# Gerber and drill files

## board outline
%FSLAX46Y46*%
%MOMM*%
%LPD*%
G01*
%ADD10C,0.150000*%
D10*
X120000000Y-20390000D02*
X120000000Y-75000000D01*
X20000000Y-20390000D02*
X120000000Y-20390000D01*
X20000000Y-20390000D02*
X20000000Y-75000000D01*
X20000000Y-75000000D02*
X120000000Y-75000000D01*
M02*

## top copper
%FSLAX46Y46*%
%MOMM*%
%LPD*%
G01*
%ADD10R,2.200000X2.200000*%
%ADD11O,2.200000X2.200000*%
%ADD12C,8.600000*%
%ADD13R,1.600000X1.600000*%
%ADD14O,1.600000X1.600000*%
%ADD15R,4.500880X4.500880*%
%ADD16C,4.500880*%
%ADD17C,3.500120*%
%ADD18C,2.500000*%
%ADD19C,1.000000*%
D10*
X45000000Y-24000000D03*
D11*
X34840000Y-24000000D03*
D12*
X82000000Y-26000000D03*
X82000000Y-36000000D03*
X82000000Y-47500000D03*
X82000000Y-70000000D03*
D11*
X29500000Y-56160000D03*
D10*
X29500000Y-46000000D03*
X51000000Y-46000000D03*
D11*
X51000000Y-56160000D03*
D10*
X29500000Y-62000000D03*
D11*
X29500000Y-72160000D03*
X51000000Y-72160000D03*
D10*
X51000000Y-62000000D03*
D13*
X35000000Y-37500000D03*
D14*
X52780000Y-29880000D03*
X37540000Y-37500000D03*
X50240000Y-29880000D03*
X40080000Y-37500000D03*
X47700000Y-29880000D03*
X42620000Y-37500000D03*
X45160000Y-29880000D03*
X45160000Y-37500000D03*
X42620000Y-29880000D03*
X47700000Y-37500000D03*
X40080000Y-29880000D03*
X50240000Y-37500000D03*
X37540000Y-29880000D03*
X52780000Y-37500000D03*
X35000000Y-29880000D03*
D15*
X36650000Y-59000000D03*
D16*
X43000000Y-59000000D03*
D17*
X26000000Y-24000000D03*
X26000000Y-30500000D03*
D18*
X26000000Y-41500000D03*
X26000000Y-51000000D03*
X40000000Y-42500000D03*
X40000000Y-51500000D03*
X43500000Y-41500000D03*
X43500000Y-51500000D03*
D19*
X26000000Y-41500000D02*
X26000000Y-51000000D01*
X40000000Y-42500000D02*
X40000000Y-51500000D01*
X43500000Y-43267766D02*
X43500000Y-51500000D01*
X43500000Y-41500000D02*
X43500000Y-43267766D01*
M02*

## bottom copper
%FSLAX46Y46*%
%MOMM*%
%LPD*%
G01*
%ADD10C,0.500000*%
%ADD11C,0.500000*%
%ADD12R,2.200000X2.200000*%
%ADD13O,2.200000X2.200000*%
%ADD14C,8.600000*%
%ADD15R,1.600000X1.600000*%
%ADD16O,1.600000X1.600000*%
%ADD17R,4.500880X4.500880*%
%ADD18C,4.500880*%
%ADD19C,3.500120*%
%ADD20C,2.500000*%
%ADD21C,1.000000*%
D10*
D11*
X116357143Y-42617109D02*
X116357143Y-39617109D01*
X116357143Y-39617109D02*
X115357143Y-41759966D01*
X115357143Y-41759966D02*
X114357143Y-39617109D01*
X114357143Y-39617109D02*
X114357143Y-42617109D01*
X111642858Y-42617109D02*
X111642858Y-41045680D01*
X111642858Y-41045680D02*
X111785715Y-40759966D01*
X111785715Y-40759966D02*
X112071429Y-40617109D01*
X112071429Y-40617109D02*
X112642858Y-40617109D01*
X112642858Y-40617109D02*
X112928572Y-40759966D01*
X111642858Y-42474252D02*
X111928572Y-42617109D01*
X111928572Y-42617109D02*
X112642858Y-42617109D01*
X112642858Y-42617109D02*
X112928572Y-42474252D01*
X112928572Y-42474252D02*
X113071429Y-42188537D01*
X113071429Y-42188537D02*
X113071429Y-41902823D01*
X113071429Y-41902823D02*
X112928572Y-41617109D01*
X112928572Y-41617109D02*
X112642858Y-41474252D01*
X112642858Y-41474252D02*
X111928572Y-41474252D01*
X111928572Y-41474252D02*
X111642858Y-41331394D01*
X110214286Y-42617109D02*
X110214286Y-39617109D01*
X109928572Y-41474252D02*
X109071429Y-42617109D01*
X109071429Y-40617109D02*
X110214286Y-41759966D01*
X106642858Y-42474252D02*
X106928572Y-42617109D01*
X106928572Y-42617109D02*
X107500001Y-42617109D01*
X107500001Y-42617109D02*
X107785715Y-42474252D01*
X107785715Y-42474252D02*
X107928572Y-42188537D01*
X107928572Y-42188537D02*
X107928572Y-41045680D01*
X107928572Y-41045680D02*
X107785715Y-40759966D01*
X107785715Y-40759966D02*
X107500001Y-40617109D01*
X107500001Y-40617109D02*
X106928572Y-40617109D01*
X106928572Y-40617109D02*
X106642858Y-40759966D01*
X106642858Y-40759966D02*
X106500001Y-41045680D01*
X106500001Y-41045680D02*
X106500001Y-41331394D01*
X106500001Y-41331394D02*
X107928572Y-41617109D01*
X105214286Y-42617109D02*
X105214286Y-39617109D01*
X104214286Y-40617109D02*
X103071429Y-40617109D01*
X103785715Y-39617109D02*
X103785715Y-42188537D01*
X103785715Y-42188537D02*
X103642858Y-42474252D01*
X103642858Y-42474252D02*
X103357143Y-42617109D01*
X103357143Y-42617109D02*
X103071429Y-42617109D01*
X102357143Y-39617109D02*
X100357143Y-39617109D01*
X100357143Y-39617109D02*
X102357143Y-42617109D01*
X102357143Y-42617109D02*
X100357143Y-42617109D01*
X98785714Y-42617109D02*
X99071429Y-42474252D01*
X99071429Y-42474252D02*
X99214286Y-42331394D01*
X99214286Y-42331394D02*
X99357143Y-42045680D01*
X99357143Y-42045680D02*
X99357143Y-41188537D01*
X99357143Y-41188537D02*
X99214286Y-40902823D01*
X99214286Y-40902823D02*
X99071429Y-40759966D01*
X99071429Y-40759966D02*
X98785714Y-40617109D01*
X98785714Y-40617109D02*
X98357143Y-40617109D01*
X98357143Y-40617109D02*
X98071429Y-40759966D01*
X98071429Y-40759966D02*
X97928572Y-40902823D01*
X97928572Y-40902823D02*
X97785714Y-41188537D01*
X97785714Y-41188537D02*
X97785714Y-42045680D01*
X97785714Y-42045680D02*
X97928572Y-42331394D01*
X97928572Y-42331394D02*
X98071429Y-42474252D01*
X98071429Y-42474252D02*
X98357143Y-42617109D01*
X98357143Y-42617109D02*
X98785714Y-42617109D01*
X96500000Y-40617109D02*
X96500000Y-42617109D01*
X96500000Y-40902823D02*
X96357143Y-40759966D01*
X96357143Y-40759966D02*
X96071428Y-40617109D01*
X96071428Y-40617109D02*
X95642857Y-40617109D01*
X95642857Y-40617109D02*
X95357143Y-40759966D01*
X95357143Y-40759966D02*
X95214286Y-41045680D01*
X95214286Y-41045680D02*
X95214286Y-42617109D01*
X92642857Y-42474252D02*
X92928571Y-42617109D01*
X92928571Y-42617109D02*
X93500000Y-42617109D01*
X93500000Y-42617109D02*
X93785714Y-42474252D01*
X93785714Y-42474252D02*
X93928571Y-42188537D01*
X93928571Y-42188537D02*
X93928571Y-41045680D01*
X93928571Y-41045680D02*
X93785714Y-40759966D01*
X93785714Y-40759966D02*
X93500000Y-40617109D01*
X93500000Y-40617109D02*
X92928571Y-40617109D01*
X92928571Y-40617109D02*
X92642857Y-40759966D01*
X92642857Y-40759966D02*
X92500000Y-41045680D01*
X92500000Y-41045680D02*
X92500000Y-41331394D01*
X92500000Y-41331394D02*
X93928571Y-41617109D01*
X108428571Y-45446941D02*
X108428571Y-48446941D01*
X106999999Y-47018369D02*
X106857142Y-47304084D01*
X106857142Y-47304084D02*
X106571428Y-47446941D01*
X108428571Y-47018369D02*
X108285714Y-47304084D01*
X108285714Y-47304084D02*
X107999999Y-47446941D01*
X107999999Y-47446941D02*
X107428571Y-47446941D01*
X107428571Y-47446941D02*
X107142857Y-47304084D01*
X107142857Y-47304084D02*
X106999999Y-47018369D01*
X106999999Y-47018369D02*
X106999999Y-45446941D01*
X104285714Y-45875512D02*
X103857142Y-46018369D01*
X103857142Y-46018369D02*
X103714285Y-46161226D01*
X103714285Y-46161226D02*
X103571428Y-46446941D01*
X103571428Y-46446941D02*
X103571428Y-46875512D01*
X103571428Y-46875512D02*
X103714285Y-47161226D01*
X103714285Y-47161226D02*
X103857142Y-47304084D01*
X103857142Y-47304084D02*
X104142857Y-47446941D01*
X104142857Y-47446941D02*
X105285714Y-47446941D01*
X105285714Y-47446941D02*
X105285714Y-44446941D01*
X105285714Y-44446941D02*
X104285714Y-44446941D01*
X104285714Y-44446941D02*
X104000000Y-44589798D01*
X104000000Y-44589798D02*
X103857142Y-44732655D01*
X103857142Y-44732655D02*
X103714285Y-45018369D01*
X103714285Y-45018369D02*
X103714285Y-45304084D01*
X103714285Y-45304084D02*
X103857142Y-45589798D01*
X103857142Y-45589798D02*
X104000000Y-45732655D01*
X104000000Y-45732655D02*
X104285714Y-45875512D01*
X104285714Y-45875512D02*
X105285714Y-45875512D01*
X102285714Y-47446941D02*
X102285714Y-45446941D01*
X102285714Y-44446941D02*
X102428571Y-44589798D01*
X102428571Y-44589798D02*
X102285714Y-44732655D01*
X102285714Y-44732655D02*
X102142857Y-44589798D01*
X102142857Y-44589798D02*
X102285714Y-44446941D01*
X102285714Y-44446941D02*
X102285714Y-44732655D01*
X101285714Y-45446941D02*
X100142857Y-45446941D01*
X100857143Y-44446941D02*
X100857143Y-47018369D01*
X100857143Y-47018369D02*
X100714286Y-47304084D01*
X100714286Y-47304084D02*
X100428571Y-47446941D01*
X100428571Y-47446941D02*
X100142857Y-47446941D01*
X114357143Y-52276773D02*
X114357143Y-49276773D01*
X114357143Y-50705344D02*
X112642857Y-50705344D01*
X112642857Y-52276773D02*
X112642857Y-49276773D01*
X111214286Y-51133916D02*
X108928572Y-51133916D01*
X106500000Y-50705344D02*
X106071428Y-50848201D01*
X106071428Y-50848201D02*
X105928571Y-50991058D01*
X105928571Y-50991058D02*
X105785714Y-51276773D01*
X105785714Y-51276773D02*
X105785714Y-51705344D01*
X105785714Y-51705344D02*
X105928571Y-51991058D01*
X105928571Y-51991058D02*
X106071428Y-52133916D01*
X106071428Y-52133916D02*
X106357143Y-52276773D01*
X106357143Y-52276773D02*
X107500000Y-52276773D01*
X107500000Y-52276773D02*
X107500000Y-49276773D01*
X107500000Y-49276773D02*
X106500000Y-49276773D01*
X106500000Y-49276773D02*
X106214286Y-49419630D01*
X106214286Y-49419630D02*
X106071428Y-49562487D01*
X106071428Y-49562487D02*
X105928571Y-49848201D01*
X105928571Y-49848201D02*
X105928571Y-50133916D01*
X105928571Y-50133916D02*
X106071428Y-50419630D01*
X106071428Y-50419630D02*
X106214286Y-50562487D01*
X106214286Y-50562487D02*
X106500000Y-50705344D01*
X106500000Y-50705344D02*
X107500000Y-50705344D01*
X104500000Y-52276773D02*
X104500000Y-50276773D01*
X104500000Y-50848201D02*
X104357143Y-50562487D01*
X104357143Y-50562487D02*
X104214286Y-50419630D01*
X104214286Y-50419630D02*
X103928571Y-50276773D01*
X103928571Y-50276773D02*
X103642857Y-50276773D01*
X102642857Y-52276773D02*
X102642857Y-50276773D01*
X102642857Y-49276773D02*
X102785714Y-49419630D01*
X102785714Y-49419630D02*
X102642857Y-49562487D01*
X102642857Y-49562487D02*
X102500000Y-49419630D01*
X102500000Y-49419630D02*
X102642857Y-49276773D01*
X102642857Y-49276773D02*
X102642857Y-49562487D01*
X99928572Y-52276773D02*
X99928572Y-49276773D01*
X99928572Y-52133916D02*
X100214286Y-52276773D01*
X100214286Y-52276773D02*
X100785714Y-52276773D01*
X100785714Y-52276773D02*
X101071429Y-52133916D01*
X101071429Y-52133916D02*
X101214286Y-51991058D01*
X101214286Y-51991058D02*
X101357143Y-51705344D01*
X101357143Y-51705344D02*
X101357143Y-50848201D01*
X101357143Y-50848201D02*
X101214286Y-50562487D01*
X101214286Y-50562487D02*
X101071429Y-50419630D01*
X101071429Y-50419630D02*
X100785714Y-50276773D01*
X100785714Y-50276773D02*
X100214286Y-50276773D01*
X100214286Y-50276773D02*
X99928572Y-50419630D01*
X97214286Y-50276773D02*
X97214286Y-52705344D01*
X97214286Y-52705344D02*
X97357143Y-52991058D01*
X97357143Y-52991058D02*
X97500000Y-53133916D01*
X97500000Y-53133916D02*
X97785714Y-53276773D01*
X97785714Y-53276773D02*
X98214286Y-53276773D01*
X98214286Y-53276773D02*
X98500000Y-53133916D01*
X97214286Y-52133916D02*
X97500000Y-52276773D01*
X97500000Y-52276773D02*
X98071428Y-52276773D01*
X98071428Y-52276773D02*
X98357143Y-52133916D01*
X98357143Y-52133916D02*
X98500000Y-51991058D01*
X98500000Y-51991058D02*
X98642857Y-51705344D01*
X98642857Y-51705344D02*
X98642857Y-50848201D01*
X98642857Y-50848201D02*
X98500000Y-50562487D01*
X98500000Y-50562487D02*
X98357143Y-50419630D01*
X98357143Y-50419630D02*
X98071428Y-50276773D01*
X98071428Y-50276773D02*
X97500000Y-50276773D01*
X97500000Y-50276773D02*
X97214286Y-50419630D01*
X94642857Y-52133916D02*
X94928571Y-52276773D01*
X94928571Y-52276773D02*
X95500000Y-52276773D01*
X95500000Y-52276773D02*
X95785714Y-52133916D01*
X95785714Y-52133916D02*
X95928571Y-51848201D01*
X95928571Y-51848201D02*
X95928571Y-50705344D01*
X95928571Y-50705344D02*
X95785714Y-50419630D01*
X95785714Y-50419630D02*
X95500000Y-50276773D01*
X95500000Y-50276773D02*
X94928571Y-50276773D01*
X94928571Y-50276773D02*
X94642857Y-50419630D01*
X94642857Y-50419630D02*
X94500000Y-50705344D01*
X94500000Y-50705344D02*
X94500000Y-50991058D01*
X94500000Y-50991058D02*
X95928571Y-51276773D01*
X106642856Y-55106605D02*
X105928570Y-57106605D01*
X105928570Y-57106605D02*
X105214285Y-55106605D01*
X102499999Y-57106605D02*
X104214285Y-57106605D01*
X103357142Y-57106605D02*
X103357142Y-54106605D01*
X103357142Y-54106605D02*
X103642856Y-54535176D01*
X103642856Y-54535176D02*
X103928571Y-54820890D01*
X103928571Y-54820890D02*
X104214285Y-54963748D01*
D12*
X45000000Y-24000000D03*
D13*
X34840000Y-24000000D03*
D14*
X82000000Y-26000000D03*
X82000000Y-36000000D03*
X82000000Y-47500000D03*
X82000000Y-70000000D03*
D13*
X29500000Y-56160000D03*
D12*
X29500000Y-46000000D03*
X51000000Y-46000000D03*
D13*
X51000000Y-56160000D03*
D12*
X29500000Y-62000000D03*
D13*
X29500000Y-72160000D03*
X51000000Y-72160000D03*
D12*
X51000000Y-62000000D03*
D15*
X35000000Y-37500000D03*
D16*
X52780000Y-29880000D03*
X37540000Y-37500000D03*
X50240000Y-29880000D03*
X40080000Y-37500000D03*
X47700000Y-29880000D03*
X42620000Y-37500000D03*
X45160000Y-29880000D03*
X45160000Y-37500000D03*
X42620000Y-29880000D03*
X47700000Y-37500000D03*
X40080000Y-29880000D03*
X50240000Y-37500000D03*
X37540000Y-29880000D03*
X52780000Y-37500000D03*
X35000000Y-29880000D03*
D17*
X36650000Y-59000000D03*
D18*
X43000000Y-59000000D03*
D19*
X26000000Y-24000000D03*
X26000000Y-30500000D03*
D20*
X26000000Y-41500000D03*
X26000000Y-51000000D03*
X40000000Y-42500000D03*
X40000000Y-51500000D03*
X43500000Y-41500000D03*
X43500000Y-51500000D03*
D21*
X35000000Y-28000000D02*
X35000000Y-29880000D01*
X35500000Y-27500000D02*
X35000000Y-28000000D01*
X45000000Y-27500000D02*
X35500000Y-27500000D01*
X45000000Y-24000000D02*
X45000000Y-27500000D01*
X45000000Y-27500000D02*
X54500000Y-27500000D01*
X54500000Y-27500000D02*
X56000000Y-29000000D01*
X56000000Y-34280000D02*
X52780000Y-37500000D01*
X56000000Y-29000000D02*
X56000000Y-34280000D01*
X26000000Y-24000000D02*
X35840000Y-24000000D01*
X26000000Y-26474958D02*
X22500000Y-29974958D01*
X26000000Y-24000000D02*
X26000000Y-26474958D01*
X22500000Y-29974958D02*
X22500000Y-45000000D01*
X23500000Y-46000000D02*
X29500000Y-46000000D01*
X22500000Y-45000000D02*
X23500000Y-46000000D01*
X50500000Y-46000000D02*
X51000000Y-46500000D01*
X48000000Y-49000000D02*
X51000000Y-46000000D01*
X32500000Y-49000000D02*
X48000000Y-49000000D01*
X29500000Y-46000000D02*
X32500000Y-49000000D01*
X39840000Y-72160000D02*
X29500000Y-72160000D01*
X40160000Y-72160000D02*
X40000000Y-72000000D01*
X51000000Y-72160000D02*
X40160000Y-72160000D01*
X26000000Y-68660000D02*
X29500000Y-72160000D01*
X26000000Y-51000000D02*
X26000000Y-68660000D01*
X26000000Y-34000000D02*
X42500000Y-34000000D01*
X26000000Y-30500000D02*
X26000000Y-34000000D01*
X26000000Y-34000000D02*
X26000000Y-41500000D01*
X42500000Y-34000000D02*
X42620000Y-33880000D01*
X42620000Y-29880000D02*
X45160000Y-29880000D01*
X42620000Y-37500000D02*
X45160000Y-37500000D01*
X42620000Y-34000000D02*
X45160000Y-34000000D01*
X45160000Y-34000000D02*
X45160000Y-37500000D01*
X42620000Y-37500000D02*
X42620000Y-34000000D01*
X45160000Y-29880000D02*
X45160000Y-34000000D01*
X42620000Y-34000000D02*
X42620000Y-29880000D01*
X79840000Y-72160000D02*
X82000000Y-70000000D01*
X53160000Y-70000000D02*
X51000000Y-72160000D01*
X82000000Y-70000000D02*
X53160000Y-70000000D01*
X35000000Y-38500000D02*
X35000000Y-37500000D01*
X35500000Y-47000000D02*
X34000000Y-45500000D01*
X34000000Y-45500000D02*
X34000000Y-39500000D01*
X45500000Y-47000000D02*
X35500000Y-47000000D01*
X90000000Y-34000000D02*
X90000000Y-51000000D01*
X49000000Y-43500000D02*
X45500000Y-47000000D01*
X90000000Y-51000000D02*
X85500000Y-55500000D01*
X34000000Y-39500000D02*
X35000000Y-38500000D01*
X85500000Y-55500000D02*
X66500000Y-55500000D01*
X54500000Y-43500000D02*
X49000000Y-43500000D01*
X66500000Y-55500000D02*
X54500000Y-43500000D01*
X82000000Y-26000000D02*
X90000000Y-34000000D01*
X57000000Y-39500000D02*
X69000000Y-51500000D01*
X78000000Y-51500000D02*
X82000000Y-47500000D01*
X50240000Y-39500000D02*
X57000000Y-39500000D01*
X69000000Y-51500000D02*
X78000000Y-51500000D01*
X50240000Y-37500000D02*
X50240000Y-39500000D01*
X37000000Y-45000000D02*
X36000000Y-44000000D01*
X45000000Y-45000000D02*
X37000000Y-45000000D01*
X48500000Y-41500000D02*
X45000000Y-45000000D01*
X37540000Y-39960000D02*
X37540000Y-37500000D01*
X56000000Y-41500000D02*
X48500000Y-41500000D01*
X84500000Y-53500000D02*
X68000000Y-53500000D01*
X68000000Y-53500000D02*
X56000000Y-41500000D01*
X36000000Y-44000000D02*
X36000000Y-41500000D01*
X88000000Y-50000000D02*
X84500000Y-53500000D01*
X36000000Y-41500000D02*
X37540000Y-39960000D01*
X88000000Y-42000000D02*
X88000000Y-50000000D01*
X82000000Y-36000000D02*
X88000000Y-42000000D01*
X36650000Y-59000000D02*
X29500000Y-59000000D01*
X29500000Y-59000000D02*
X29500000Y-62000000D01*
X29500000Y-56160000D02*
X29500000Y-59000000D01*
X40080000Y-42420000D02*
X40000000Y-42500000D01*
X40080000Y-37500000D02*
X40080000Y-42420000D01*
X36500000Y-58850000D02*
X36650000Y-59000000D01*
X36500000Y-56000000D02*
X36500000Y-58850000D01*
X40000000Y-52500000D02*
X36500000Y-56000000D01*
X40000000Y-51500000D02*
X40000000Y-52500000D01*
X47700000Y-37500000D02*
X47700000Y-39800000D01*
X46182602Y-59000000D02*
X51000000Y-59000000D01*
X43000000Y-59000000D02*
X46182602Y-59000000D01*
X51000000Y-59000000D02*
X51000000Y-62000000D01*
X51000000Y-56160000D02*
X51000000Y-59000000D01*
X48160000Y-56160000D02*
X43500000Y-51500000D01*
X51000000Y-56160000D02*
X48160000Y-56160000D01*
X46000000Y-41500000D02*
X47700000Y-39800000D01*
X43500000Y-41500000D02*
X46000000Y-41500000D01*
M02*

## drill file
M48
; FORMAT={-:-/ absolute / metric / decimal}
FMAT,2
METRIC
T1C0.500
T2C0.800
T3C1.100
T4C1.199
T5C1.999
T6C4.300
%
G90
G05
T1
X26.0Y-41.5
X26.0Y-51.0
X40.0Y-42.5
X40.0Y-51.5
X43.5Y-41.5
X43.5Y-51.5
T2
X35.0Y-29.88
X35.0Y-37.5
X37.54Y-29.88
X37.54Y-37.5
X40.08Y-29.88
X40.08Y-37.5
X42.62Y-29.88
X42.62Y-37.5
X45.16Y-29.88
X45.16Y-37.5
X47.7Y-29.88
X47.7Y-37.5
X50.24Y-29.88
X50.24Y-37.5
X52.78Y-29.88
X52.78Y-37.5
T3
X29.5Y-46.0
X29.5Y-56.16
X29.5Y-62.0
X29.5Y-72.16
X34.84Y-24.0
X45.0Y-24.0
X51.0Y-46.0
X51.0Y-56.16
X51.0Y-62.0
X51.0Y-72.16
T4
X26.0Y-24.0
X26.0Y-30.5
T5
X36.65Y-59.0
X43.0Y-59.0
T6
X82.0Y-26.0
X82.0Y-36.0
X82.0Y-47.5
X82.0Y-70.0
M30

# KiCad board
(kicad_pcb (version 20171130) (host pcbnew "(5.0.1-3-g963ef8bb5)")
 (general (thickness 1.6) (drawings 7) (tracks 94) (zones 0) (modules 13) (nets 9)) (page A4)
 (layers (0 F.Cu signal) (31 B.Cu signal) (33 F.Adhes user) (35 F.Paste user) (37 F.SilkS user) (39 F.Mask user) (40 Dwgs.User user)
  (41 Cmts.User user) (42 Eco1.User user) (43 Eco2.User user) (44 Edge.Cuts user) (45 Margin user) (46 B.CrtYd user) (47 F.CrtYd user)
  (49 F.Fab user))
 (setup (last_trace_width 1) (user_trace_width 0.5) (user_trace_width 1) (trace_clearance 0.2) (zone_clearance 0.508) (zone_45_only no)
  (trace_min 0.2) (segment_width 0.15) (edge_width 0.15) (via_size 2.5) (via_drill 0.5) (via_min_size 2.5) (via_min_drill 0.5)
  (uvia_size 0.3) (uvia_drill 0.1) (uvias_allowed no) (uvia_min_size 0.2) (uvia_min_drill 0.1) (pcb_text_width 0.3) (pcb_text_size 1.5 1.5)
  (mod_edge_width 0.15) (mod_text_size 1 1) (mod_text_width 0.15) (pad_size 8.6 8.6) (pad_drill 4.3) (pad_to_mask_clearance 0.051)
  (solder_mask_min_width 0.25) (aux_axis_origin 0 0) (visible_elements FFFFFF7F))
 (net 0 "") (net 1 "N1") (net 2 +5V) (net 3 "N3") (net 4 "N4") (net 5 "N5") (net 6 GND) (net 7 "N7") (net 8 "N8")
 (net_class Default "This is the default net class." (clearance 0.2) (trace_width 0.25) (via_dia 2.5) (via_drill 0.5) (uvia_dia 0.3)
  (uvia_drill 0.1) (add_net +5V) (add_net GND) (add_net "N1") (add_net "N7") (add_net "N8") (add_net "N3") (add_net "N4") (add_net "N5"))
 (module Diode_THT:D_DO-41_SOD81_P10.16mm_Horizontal (layer F.Cu) (at 45 24 180)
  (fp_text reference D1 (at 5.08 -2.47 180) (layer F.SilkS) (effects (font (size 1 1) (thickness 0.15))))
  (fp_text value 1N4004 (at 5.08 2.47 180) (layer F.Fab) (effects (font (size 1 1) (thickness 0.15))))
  (pad 1 thru_hole rect (at 0 0 180) (size 2.2 2.2) (drill 1.1) (layers *.Cu *.Mask) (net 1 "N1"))
  (pad 2 thru_hole oval (at 10.16 0 180) (size 2.2 2.2) (drill 1.1) (layers *.Cu *.Mask) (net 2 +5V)))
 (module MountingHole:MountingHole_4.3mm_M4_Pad (layer F.Cu) (at 82 26)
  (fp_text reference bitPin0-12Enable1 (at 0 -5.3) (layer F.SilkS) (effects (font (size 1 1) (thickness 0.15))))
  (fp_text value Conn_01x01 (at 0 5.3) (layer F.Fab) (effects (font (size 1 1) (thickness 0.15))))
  (pad 1 thru_hole circle (at 0 0) (size 8.6 8.6) (drill 4.3) (layers *.Cu *.Mask) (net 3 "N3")))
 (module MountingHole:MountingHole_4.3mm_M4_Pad (layer F.Cu) (at 82 36)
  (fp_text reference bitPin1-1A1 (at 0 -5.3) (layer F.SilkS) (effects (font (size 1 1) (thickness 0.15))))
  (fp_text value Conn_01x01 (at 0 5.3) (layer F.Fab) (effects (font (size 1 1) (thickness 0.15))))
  (pad 1 thru_hole circle (at 0 0) (size 8.6 8.6) (drill 4.3) (layers *.Cu *.Mask) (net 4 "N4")))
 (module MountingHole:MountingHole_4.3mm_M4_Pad (layer F.Cu) (at 82 47.5)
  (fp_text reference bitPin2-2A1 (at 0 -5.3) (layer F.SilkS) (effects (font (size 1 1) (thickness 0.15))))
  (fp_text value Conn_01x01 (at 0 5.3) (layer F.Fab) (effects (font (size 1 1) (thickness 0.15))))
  (pad 1 thru_hole circle (at 0 0) (size 8.6 8.6) (drill 4.3) (layers *.Cu *.Mask) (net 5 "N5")))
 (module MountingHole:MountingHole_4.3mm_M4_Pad (layer F.Cu) (at 82 70)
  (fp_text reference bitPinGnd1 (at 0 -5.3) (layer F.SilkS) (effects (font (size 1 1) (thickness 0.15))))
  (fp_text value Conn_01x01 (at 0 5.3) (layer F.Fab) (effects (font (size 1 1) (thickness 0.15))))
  (pad 1 thru_hole circle (at 0 0) (size 8.6 8.6) (drill 4.3) (layers *.Cu *.Mask) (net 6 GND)))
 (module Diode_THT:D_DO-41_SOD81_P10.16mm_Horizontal (layer F.Cu) (at 29.5 46 270)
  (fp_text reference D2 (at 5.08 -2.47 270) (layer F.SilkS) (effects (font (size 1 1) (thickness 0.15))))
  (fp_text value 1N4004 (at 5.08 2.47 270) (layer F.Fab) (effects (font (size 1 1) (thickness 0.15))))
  (pad 2 thru_hole oval (at 10.16 0 270) (size 2.2 2.2) (drill 1.1) (layers *.Cu *.Mask) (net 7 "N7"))
  (pad 1 thru_hole rect (at 0 0 270) (size 2.2 2.2) (drill 1.1) (layers *.Cu *.Mask) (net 2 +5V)))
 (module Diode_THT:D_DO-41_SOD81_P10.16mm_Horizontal (layer F.Cu) (at 51 46 270)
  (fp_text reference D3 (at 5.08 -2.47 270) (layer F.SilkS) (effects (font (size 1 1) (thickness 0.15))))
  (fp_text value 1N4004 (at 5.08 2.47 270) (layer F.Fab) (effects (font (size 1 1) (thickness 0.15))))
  (pad 1 thru_hole rect (at 0 0 270) (size 2.2 2.2) (drill 1.1) (layers *.Cu *.Mask) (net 2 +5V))
  (pad 2 thru_hole oval (at 10.16 0 270) (size 2.2 2.2) (drill 1.1) (layers *.Cu *.Mask) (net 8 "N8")))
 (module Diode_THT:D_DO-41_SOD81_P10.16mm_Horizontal (layer F.Cu) (at 29.5 62 270)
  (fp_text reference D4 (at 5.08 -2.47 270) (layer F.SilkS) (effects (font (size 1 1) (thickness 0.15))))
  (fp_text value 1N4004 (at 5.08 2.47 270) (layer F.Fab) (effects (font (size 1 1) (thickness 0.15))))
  (pad 1 thru_hole rect (at 0 0 270) (size 2.2 2.2) (drill 1.1) (layers *.Cu *.Mask) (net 7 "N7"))
  (pad 2 thru_hole oval (at 10.16 0 270) (size 2.2 2.2) (drill 1.1) (layers *.Cu *.Mask) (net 6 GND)))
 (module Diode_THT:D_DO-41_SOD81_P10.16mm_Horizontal (layer F.Cu) (at 51 62 270)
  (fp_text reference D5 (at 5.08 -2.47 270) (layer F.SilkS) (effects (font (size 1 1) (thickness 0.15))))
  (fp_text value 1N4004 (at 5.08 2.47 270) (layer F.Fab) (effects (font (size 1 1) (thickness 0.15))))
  (pad 2 thru_hole oval (at 10.16 0 270) (size 2.2 2.2) (drill 1.1) (layers *.Cu *.Mask) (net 6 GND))
  (pad 1 thru_hole rect (at 0 0 270) (size 2.2 2.2) (drill 1.1) (layers *.Cu *.Mask) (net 8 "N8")))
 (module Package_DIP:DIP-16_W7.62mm (layer F.Cu) (at 35 37.5 90)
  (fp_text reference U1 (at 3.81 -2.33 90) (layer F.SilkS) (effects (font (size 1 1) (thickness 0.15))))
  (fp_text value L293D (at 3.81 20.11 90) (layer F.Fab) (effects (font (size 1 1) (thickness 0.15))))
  (pad 1 thru_hole rect (at 0 0 90) (size 1.6 1.6) (drill 0.8) (layers *.Cu *.Mask) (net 3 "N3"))
  (pad 9 thru_hole oval (at 7.62 17.78 90) (size 1.6 1.6) (drill 0.8) (layers *.Cu *.Mask) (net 6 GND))
  (pad 2 thru_hole oval (at 0 2.54 90) (size 1.6 1.6) (drill 0.8) (layers *.Cu *.Mask) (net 4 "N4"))
  (pad 10 thru_hole oval (at 7.62 15.24 90) (size 1.6 1.6) (drill 0.8) (layers *.Cu *.Mask))
  (pad 3 thru_hole oval (at 0 5.08 90) (size 1.6 1.6) (drill 0.8) (layers *.Cu *.Mask) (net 7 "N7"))
  (pad 11 thru_hole oval (at 7.62 12.7 90) (size 1.6 1.6) (drill 0.8) (layers *.Cu *.Mask))
  (pad 4 thru_hole oval (at 0 7.62 90) (size 1.6 1.6) (drill 0.8) (layers *.Cu *.Mask) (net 6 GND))
  (pad 12 thru_hole oval (at 7.62 10.16 90) (size 1.6 1.6) (drill 0.8) (layers *.Cu *.Mask) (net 6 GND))
  (pad 5 thru_hole oval (at 0 10.16 90) (size 1.6 1.6) (drill 0.8) (layers *.Cu *.Mask) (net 6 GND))
  (pad 13 thru_hole oval (at 7.62 7.62 90) (size 1.6 1.6) (drill 0.8) (layers *.Cu *.Mask) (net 6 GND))
  (pad 6 thru_hole oval (at 0 12.7 90) (size 1.6 1.6) (drill 0.8) (layers *.Cu *.Mask) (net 8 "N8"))
  (pad 14 thru_hole oval (at 7.62 5.08 90) (size 1.6 1.6) (drill 0.8) (layers *.Cu *.Mask))
  (pad 7 thru_hole oval (at 0 15.24 90) (size 1.6 1.6) (drill 0.8) (layers *.Cu *.Mask) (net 5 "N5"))
  (pad 15 thru_hole oval (at 7.62 2.54 90) (size 1.6 1.6) (drill 0.8) (layers *.Cu *.Mask))
  (pad 8 thru_hole oval (at 0 17.78 90) (size 1.6 1.6) (drill 0.8) (layers *.Cu *.Mask) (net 1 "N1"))
  (pad 16 thru_hole oval (at 7.62 0 90) (size 1.6 1.6) (drill 0.8) (layers *.Cu *.Mask) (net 1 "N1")))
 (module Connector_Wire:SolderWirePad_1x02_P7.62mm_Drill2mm (layer F.Cu) (at 36.65 59)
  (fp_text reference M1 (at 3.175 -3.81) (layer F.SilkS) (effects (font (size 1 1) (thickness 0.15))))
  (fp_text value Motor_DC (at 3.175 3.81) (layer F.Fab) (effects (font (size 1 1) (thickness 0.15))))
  (pad 1 thru_hole rect (at 0 0) (size 4.50088 4.50088) (drill 1.99898) (layers *.Cu *.Mask) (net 7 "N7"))
  (pad 2 thru_hole circle (at 6.35 0) (size 4.50088 4.50088) (drill 1.99898) (layers *.Cu *.Mask) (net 8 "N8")))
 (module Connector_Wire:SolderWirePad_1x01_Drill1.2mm (layer F.Cu) (at 26 24 270)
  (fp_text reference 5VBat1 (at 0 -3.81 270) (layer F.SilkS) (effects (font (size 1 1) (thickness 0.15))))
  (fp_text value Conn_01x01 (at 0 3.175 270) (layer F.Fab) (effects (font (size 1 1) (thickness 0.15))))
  (pad 1 thru_hole circle (at 0 0 270) (size 3.50012 3.50012) (drill 1.19888) (layers *.Cu *.Mask) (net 2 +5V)))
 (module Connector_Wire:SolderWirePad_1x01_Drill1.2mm (layer F.Cu) (at 26 30.5 270)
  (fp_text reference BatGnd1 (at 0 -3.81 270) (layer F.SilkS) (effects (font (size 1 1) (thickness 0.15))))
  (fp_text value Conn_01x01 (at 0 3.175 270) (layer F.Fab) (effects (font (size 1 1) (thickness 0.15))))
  (pad 1 thru_hole circle (at 0 0 270) (size 3.50012 3.50012) (drill 1.19888) (layers *.Cu *.Mask) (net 6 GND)))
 (gr_line (start 120 20.39) (end 120 75) (layer Edge.Cuts) (width 0.15))
 (gr_line (start 20 20.39) (end 120 20.39) (layer Edge.Cuts) (width 0.15))
 (gr_line (start 20 20.39) (end 20 75) (layer Edge.Cuts) (width 0.15))
 (gr_line (start 20 75) (end 120 75) (layer Edge.Cuts) (width 0.15))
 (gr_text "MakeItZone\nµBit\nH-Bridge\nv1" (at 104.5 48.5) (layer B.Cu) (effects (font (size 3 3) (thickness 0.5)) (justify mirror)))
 (segment (start 35 28) (end 35 29.88) (width 1) (layer B.Cu) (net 1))
 (segment (start 35.5 27.5) (end 35 28) (width 1) (layer B.Cu) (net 1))
 (segment (start 45 27.5) (end 35.5 27.5) (width 1) (layer B.Cu) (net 1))
 (segment (start 45 24) (end 45 27.5) (width 1) (layer B.Cu) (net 1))
 (segment (start 45 27.5) (end 54.5 27.5) (width 1) (layer B.Cu) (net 1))
 (segment (start 54.5 27.5) (end 56 29) (width 1) (layer B.Cu) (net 1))
 (segment (start 56 34.28) (end 52.78 37.5) (width 1) (layer B.Cu) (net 1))
 (segment (start 56 29) (end 56 34.28) (width 1) (layer B.Cu) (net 1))
 (segment (start 26 24) (end 35.84 24) (width 1) (layer B.Cu) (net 2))
 (segment (start 26 26.474958) (end 22.5 29.974958) (width 1) (layer B.Cu) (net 2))
 (segment (start 26 24) (end 26 26.474958) (width 1) (layer B.Cu) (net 2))
 (segment (start 22.5 29.974958) (end 22.5 45) (width 1) (layer B.Cu) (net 2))
 (segment (start 23.5 46) (end 29.5 46) (width 1) (layer B.Cu) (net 2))
 (segment (start 22.5 45) (end 23.5 46) (width 1) (layer B.Cu) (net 2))
 (segment (start 50.5 46) (end 51 46.5) (width 1) (layer B.Cu) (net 2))
 (segment (start 48 49) (end 51 46) (width 1) (layer B.Cu) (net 2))
 (segment (start 32.5 49) (end 48 49) (width 1) (layer B.Cu) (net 2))
 (segment (start 29.5 46) (end 32.5 49) (width 1) (layer B.Cu) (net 2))
 (segment (start 39.84 72.16) (end 29.5 72.16) (width 1) (layer B.Cu) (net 6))
 (segment (start 40.16 72.16) (end 40 72) (width 1) (layer B.Cu) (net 6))
 (segment (start 51 72.16) (end 40.16 72.16) (width 1) (layer B.Cu) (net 6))
 (via (at 26 41.5) (size 2.5) (drill 0.5) (layers F.Cu B.Cu) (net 6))
 (via (at 26 51) (size 2.5) (drill 0.5) (layers F.Cu B.Cu) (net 6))
 (segment (start 26 41.5) (end 26 51) (width 1) (layer F.Cu) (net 6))
 (segment (start 26 68.66) (end 29.5 72.16) (width 1) (layer B.Cu) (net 6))
 (segment (start 26 51) (end 26 68.66) (width 1) (layer B.Cu) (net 6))
 (segment (start 26 34) (end 42.5 34) (width 1) (layer B.Cu) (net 6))
 (segment (start 26 30.5) (end 26 34) (width 1) (layer B.Cu) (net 6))
 (segment (start 26 34) (end 26 41.5) (width 1) (layer B.Cu) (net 6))
 (segment (start 42.5 34) (end 42.62 33.88) (width 1) (layer B.Cu) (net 6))
 (segment (start 42.62 29.88) (end 45.16 29.88) (width 1) (layer B.Cu) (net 6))
 (segment (start 42.62 37.5) (end 45.16 37.5) (width 1) (layer B.Cu) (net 6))
 (segment (start 42.62 34) (end 45.16 34) (width 1) (layer B.Cu) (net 6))
 (segment (start 45.16 34) (end 45.16 37.5) (width 1) (layer B.Cu) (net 6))
 (segment (start 42.62 37.5) (end 42.62 34) (width 1) (layer B.Cu) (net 6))
 (segment (start 45.16 29.88) (end 45.16 34) (width 1) (layer B.Cu) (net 6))
 (segment (start 42.62 34) (end 42.62 29.88) (width 1) (layer B.Cu) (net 6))
 (segment (start 79.84 72.16) (end 82 70) (width 1) (layer B.Cu) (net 6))
 (segment (start 53.16 70) (end 51 72.16) (width 1) (layer B.Cu) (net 6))
 (segment (start 82 70) (end 53.16 70) (width 1) (layer B.Cu) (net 6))
 (segment (start 35 38.5) (end 35 37.5) (width 1) (layer B.Cu) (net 3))
 (segment (start 35.5 47) (end 34 45.5) (width 1) (layer B.Cu) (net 3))
 (segment (start 34 45.5) (end 34 39.5) (width 1) (layer B.Cu) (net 3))
 (segment (start 45.5 47) (end 35.5 47) (width 1) (layer B.Cu) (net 3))
 (segment (start 90 34) (end 90 51) (width 1) (layer B.Cu) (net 3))
 (segment (start 49 43.5) (end 45.5 47) (width 1) (layer B.Cu) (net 3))
 (segment (start 90 51) (end 85.5 55.5) (width 1) (layer B.Cu) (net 3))
 (segment (start 34 39.5) (end 35 38.5) (width 1) (layer B.Cu) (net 3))
 (segment (start 85.5 55.5) (end 66.5 55.5) (width 1) (layer B.Cu) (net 3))
 (segment (start 54.5 43.5) (end 49 43.5) (width 1) (layer B.Cu) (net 3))
 (segment (start 66.5 55.5) (end 54.5 43.5) (width 1) (layer B.Cu) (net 3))
 (segment (start 82 26) (end 90 34) (width 1) (layer B.Cu) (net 3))
 (segment (start 57 39.5) (end 69 51.5) (width 1) (layer B.Cu) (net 5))
 (segment (start 78 51.5) (end 82 47.5) (width 1) (layer B.Cu) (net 5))
 (segment (start 50.24 39.5) (end 57 39.5) (width 1) (layer B.Cu) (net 5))
 (segment (start 69 51.5) (end 78 51.5) (width 1) (layer B.Cu) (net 5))
 (segment (start 50.24 37.5) (end 50.24 39.5) (width 1) (layer B.Cu) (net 5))
 (segment (start 37 45) (end 36 44) (width 1) (layer B.Cu) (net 4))
 (segment (start 45 45) (end 37 45) (width 1) (layer B.Cu) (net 4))
 (segment (start 48.5 41.5) (end 45 45) (width 1) (layer B.Cu) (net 4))
 (segment (start 37.54 39.96) (end 37.54 37.5) (width 1) (layer B.Cu) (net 4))
 (segment (start 56 41.5) (end 48.5 41.5) (width 1) (layer B.Cu) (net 4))
 (segment (start 84.5 53.5) (end 68 53.5) (width 1) (layer B.Cu) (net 4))
 (segment (start 68 53.5) (end 56 41.5) (width 1) (layer B.Cu) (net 4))
 (segment (start 36 44) (end 36 41.5) (width 1) (layer B.Cu) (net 4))
 (segment (start 88 50) (end 84.5 53.5) (width 1) (layer B.Cu) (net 4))
 (segment (start 36 41.5) (end 37.54 39.96) (width 1) (layer B.Cu) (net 4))
 (segment (start 88 42) (end 88 50) (width 1) (layer B.Cu) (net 4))
 (segment (start 82 36) (end 88 42) (width 1) (layer B.Cu) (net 4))
 (segment (start 36.65 59) (end 29.5 59) (width 1) (layer B.Cu) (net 7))
 (segment (start 29.5 59) (end 29.5 62) (width 1) (layer B.Cu) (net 7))
 (segment (start 29.5 56.16) (end 29.5 59) (width 1) (layer B.Cu) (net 7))
 (via (at 40 42.5) (size 2.5) (drill 0.5) (layers F.Cu B.Cu) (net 7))
 (segment (start 40.08 42.42) (end 40 42.5) (width 1) (layer B.Cu) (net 7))
 (segment (start 40.08 37.5) (end 40.08 42.42) (width 1) (layer B.Cu) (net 7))
 (via (at 40 51.5) (size 2.5) (drill 0.5) (layers F.Cu B.Cu) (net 7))
 (segment (start 40 42.5) (end 40 51.5) (width 1) (layer F.Cu) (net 7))
 (segment (start 36.5 58.85) (end 36.65 59) (width 1) (layer B.Cu) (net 7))
 (segment (start 36.5 56) (end 36.5 58.85) (width 1) (layer B.Cu) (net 7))
 (segment (start 40 52.5) (end 36.5 56) (width 1) (layer B.Cu) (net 7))
 (segment (start 40 51.5) (end 40 52.5) (width 1) (layer B.Cu) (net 7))
 (via (at 43.5 41.5) (size 2.5) (drill 0.5) (layers F.Cu B.Cu) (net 8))
 (segment (start 47.7 37.5) (end 47.7 39.8) (width 1) (layer B.Cu) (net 8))
 (via (at 43.5 51.5) (size 2.5) (drill 0.5) (layers F.Cu B.Cu) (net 8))
 (segment (start 46.182602 59) (end 51 59) (width 1) (layer B.Cu) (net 8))
 (segment (start 43 59) (end 46.182602 59) (width 1) (layer B.Cu) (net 8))
 (segment (start 51 59) (end 51 62) (width 1) (layer B.Cu) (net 8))
 (segment (start 51 56.16) (end 51 59) (width 1) (layer B.Cu) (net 8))
 (segment (start 48.16 56.16) (end 43.5 51.5) (width 1) (layer B.Cu) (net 8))
 (segment (start 51 56.16) (end 48.16 56.16) (width 1) (layer B.Cu) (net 8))
 (segment (start 46 41.5) (end 47.7 39.8) (width 1) (layer B.Cu) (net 8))
 (segment (start 43.5 41.5) (end 46 41.5) (width 1) (layer B.Cu) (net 8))
 (segment (start 43.5 43.267766) (end 43.5 51.5) (width 1) (layer F.Cu) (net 8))
 (segment (start 43.5 41.5) (end 43.5 43.267766) (width 1) (layer F.Cu) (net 8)))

